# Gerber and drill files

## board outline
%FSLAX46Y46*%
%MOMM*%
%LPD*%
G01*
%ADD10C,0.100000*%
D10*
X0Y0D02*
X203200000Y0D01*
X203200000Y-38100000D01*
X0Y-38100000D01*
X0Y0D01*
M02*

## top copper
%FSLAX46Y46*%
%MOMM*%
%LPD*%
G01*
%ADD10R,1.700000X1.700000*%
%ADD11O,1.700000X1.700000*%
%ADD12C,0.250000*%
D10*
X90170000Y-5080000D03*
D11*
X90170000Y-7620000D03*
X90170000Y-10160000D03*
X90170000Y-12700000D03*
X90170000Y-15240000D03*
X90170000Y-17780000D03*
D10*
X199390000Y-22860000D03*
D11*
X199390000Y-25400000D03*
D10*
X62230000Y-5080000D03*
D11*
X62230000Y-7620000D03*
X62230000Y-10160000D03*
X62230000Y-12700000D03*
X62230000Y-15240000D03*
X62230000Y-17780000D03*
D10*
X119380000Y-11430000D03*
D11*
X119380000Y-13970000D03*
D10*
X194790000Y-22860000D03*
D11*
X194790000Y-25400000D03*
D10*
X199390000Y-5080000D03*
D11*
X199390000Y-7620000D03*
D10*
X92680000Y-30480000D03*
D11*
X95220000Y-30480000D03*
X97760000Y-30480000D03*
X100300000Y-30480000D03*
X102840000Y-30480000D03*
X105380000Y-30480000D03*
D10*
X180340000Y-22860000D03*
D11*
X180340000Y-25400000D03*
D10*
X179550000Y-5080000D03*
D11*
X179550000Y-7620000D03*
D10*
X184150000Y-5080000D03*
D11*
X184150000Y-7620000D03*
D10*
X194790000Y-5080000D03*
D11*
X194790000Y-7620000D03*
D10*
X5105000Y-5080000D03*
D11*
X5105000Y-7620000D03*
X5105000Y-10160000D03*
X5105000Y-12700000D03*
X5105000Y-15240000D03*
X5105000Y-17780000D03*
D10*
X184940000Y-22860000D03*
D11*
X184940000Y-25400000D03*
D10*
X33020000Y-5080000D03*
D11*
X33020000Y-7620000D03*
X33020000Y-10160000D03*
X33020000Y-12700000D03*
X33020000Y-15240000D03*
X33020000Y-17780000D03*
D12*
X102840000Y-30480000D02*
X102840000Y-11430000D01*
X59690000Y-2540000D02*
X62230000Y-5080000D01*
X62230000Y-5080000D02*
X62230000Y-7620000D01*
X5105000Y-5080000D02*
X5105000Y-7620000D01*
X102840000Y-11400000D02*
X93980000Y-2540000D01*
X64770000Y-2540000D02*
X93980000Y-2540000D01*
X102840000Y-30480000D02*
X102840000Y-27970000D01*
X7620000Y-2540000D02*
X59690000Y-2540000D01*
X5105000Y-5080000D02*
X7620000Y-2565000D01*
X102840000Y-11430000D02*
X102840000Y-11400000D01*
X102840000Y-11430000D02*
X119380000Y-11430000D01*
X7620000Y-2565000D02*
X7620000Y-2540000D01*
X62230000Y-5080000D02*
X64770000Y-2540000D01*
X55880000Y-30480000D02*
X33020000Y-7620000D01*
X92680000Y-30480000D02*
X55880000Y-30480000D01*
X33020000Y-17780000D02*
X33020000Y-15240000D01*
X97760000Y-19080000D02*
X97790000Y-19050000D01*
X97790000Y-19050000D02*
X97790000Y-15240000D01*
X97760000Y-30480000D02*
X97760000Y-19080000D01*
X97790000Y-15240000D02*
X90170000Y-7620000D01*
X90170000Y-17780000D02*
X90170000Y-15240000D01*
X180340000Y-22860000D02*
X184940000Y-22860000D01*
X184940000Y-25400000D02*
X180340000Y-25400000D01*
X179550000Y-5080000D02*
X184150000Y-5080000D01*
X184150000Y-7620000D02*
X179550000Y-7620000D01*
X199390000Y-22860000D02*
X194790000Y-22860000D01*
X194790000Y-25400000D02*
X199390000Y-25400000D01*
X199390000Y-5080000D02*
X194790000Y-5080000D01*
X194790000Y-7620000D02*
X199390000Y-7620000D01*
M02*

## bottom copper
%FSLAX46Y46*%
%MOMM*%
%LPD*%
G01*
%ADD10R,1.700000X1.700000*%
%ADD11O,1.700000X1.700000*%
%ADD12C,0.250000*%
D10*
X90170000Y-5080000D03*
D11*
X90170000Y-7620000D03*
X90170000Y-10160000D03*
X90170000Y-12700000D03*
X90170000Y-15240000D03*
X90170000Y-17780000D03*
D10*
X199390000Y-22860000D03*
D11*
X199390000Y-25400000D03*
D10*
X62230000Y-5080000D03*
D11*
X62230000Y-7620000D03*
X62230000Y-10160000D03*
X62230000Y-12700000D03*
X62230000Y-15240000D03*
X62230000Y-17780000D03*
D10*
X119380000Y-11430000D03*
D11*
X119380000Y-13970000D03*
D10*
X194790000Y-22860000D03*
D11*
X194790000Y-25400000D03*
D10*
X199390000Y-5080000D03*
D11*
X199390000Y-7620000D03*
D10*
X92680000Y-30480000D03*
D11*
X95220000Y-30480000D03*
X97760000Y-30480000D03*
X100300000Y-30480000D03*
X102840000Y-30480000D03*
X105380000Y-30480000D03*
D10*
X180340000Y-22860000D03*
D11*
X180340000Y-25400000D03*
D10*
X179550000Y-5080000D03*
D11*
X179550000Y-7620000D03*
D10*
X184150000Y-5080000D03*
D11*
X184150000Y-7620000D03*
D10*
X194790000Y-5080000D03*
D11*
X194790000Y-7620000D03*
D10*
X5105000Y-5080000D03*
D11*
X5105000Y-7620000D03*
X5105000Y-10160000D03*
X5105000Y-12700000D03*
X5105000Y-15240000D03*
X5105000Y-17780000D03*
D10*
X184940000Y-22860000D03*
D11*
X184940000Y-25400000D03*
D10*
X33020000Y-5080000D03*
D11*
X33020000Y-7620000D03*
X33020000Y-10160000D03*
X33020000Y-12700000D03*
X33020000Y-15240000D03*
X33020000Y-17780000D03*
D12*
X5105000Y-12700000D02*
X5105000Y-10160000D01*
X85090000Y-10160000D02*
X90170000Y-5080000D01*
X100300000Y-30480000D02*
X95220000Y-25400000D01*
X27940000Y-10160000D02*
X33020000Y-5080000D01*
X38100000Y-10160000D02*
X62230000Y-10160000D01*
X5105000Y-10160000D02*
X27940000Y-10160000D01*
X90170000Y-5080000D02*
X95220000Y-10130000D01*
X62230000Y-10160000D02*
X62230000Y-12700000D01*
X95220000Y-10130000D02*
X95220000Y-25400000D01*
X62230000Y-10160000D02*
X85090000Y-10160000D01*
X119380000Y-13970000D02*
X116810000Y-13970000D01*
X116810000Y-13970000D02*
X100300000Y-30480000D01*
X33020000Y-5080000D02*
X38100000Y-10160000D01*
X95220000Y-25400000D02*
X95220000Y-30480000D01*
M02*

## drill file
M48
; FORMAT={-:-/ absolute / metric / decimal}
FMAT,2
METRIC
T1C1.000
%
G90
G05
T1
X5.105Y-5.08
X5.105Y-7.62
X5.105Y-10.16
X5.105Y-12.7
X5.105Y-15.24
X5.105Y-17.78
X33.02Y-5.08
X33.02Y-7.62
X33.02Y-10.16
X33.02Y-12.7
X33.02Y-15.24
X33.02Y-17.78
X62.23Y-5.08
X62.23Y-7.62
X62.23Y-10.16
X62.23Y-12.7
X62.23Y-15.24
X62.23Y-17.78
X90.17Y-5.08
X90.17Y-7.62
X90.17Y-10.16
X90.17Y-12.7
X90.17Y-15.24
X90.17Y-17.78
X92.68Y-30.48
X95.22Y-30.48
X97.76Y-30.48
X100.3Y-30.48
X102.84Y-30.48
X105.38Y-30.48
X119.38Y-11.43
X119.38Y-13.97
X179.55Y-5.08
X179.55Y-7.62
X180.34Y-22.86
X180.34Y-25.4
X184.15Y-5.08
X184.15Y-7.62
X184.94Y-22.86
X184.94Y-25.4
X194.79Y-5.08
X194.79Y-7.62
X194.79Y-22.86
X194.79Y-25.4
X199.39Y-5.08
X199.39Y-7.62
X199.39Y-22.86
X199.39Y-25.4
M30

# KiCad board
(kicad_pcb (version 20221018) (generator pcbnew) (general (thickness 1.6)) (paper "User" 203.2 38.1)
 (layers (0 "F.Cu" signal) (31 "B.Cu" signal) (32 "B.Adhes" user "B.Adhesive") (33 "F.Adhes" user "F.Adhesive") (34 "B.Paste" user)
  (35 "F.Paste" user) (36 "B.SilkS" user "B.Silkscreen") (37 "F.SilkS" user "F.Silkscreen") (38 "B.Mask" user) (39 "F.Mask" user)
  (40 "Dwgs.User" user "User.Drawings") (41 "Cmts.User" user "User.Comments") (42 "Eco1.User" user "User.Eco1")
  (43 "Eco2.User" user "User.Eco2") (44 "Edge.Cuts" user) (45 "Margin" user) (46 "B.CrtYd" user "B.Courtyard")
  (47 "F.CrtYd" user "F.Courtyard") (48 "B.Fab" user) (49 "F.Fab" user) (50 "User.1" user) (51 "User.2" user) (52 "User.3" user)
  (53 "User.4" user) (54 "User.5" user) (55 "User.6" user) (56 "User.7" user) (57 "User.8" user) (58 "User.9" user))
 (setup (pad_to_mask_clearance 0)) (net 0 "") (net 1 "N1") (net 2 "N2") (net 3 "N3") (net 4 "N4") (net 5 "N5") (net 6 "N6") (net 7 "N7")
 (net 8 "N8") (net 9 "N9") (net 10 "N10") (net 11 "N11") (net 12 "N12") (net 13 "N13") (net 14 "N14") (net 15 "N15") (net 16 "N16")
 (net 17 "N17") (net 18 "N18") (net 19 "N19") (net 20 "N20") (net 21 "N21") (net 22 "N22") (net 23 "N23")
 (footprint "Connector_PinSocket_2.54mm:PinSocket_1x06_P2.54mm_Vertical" (layer "F.Cu") (at 90.17 5.08)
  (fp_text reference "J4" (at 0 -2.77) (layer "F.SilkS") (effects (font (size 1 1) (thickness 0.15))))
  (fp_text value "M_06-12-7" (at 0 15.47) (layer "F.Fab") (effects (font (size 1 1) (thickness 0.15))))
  (pad "1" thru_hole rect (at 0 0) (size 1.7 1.7) (drill 1) (layers "*.Cu" "*.Mask") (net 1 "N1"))
  (pad "2" thru_hole oval (at 0 2.54) (size 1.7 1.7) (drill 1) (layers "*.Cu" "*.Mask") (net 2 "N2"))
  (pad "3" thru_hole oval (at 0 5.08) (size 1.7 1.7) (drill 1) (layers "*.Cu" "*.Mask") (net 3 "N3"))
  (pad "4" thru_hole oval (at 0 7.62) (size 1.7 1.7) (drill 1) (layers "*.Cu" "*.Mask") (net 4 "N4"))
  (pad "5" thru_hole oval (at 0 10.16) (size 1.7 1.7) (drill 1) (layers "*.Cu" "*.Mask") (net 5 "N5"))
  (pad "6" thru_hole oval (at 0 12.7) (size 1.7 1.7) (drill 1) (layers "*.Cu" "*.Mask") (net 5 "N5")))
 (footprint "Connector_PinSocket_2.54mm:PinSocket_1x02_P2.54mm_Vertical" (layer "F.Cu") (at 199.39 22.86)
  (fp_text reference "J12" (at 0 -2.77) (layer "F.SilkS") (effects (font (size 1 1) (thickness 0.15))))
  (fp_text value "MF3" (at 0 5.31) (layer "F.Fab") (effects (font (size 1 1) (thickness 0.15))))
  (pad "1" thru_hole rect (at 0 0) (size 1.7 1.7) (drill 1) (layers "*.Cu" "*.Mask") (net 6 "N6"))
  (pad "2" thru_hole oval (at 0 2.54) (size 1.7 1.7) (drill 1) (layers "*.Cu" "*.Mask") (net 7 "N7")))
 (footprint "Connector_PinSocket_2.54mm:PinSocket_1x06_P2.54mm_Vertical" (layer "F.Cu") (at 62.23 5.08)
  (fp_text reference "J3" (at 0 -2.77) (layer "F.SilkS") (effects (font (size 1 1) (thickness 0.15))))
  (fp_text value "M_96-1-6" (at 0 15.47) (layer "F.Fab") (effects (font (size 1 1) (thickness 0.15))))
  (pad "1" thru_hole rect (at 0 0) (size 1.7 1.7) (drill 1) (layers "*.Cu" "*.Mask") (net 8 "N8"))
  (pad "2" thru_hole oval (at 0 2.54) (size 1.7 1.7) (drill 1) (layers "*.Cu" "*.Mask") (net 8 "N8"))
  (pad "3" thru_hole oval (at 0 5.08) (size 1.7 1.7) (drill 1) (layers "*.Cu" "*.Mask") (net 1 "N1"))
  (pad "4" thru_hole oval (at 0 7.62) (size 1.7 1.7) (drill 1) (layers "*.Cu" "*.Mask") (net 1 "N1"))
  (pad "5" thru_hole oval (at 0 10.16) (size 1.7 1.7) (drill 1) (layers "*.Cu" "*.Mask") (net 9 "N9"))
  (pad "6" thru_hole oval (at 0 12.7) (size 1.7 1.7) (drill 1) (layers "*.Cu" "*.Mask") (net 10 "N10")))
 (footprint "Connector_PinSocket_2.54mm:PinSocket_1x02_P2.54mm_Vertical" (layer "F.Cu") (at 119.38 11.43)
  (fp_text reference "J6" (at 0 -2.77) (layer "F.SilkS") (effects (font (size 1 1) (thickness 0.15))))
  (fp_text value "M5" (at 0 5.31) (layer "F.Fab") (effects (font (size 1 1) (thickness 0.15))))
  (pad "1" thru_hole rect (at 0 0) (size 1.7 1.7) (drill 1) (layers "*.Cu" "*.Mask") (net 8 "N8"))
  (pad "2" thru_hole oval (at 0 2.54) (size 1.7 1.7) (drill 1) (layers "*.Cu" "*.Mask") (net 1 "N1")))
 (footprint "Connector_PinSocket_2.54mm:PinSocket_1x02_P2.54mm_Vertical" (layer "F.Cu") (at 194.79 22.86)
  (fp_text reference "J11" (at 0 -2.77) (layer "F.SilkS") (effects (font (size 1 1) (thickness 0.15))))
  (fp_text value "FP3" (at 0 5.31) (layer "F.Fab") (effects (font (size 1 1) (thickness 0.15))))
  (pad "1" thru_hole rect (at 0 0) (size 1.7 1.7) (drill 1) (layers "*.Cu" "*.Mask") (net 6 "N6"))
  (pad "2" thru_hole oval (at 0 2.54) (size 1.7 1.7) (drill 1) (layers "*.Cu" "*.Mask") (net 7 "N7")))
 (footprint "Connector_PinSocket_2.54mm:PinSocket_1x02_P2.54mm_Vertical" (layer "F.Cu") (at 199.39 5.08)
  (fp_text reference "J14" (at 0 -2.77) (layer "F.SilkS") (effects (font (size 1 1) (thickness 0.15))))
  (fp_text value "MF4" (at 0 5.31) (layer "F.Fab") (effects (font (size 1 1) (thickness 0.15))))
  (pad "1" thru_hole rect (at 0 0) (size 1.7 1.7) (drill 1) (layers "*.Cu" "*.Mask") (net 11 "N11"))
  (pad "2" thru_hole oval (at 0 2.54) (size 1.7 1.7) (drill 1) (layers "*.Cu" "*.Mask") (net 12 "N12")))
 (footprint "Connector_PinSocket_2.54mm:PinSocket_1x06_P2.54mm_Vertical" (layer "F.Cu") (at 92.68 30.48 90)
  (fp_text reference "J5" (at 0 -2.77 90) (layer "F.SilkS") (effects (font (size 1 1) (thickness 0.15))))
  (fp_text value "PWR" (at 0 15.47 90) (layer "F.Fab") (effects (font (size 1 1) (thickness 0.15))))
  (pad "1" thru_hole rect (at 0 0 90) (size 1.7 1.7) (drill 1) (layers "*.Cu" "*.Mask") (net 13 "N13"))
  (pad "2" thru_hole oval (at 0 2.54 90) (size 1.7 1.7) (drill 1) (layers "*.Cu" "*.Mask") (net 1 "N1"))
  (pad "3" thru_hole oval (at 0 5.08 90) (size 1.7 1.7) (drill 1) (layers "*.Cu" "*.Mask") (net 2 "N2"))
  (pad "4" thru_hole oval (at 0 7.62 90) (size 1.7 1.7) (drill 1) (layers "*.Cu" "*.Mask") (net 1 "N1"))
  (pad "5" thru_hole oval (at 0 10.16 90) (size 1.7 1.7) (drill 1) (layers "*.Cu" "*.Mask") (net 8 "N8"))
  (pad "6" thru_hole oval (at 0 12.7 90) (size 1.7 1.7) (drill 1) (layers "*.Cu" "*.Mask") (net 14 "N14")))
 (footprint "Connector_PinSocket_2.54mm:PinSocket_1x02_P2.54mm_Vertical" (layer "F.Cu") (at 180.34 22.86)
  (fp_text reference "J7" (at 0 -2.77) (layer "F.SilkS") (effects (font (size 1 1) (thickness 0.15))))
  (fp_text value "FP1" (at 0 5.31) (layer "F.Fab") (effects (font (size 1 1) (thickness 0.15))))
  (pad "1" thru_hole rect (at 0 0) (size 1.7 1.7) (drill 1) (layers "*.Cu" "*.Mask") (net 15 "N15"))
  (pad "2" thru_hole oval (at 0 2.54) (size 1.7 1.7) (drill 1) (layers "*.Cu" "*.Mask") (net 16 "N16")))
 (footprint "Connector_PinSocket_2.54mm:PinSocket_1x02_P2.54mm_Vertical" (layer "F.Cu") (at 179.55 5.08)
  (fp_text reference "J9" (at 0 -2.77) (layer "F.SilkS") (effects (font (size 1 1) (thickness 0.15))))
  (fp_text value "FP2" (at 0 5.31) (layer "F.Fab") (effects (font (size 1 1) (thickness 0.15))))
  (pad "1" thru_hole rect (at 0 0) (size 1.7 1.7) (drill 1) (layers "*.Cu" "*.Mask") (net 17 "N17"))
  (pad "2" thru_hole oval (at 0 2.54) (size 1.7 1.7) (drill 1) (layers "*.Cu" "*.Mask") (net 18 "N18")))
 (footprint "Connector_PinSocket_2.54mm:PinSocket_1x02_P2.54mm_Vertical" (layer "F.Cu") (at 184.15 5.08)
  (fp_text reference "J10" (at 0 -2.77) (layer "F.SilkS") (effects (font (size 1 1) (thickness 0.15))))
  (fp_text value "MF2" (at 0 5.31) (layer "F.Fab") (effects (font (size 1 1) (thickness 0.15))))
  (pad "1" thru_hole rect (at 0 0) (size 1.7 1.7) (drill 1) (layers "*.Cu" "*.Mask") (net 17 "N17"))
  (pad "2" thru_hole oval (at 0 2.54) (size 1.7 1.7) (drill 1) (layers "*.Cu" "*.Mask") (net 18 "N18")))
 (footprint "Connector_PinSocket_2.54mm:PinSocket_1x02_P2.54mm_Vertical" (layer "F.Cu") (at 194.79 5.08)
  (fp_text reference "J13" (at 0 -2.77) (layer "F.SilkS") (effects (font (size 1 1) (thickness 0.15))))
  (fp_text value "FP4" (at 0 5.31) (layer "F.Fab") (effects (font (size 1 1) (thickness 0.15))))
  (pad "1" thru_hole rect (at 0 0) (size 1.7 1.7) (drill 1) (layers "*.Cu" "*.Mask") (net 11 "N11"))
  (pad "2" thru_hole oval (at 0 2.54) (size 1.7 1.7) (drill 1) (layers "*.Cu" "*.Mask") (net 12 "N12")))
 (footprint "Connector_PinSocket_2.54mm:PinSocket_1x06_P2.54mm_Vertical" (layer "F.Cu") (at 5.105 5.08)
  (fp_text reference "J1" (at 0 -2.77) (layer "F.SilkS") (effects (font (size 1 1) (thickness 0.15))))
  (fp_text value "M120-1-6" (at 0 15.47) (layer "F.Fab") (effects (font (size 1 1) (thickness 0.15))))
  (pad "1" thru_hole rect (at 0 0) (size 1.7 1.7) (drill 1) (layers "*.Cu" "*.Mask") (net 8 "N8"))
  (pad "2" thru_hole oval (at 0 2.54) (size 1.7 1.7) (drill 1) (layers "*.Cu" "*.Mask") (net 8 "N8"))
  (pad "3" thru_hole oval (at 0 5.08) (size 1.7 1.7) (drill 1) (layers "*.Cu" "*.Mask") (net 1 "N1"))
  (pad "4" thru_hole oval (at 0 7.62) (size 1.7 1.7) (drill 1) (layers "*.Cu" "*.Mask") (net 1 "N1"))
  (pad "5" thru_hole oval (at 0 10.16) (size 1.7 1.7) (drill 1) (layers "*.Cu" "*.Mask") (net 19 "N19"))
  (pad "6" thru_hole oval (at 0 12.7) (size 1.7 1.7) (drill 1) (layers "*.Cu" "*.Mask") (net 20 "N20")))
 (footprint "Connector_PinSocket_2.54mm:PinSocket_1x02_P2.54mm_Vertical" (layer "F.Cu") (at 184.94 22.86)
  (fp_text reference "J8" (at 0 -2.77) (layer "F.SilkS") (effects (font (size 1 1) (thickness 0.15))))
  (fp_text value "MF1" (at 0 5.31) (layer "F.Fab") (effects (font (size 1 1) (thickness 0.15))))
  (pad "1" thru_hole rect (at 0 0) (size 1.7 1.7) (drill 1) (layers "*.Cu" "*.Mask") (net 15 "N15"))
  (pad "2" thru_hole oval (at 0 2.54) (size 1.7 1.7) (drill 1) (layers "*.Cu" "*.Mask") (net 16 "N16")))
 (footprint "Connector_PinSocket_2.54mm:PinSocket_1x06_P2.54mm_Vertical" (layer "F.Cu") (at 33.02 5.08)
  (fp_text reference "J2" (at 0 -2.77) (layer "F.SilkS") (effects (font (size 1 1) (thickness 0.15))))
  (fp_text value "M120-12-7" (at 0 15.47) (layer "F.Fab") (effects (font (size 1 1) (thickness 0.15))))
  (pad "1" thru_hole rect (at 0 0) (size 1.7 1.7) (drill 1) (layers "*.Cu" "*.Mask") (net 1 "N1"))
  (pad "2" thru_hole oval (at 0 2.54) (size 1.7 1.7) (drill 1) (layers "*.Cu" "*.Mask") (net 13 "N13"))
  (pad "3" thru_hole oval (at 0 5.08) (size 1.7 1.7) (drill 1) (layers "*.Cu" "*.Mask") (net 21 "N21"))
  (pad "4" thru_hole oval (at 0 7.62) (size 1.7 1.7) (drill 1) (layers "*.Cu" "*.Mask") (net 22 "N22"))
  (pad "5" thru_hole oval (at 0 10.16) (size 1.7 1.7) (drill 1) (layers "*.Cu" "*.Mask") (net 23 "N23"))
  (pad "6" thru_hole oval (at 0 12.7) (size 1.7 1.7) (drill 1) (layers "*.Cu" "*.Mask") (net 23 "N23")))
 (gr_rect (start 0 0) (end 203.2 38.1) (stroke (width 0.1) (type default)) (fill none) (layer "Edge.Cuts"))
 (segment (start 102.84 30.48) (end 102.84 11.43) (width 0.25) (layer "F.Cu") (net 8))
 (segment (start 59.69 2.54) (end 62.23 5.08) (width 0.25) (layer "F.Cu") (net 8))
 (segment (start 62.23 5.08) (end 62.23 7.62) (width 0.25) (layer "F.Cu") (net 8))
 (segment (start 5.105 5.08) (end 5.105 7.62) (width 0.25) (layer "F.Cu") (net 8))
 (segment (start 102.84 11.4) (end 93.98 2.54) (width 0.25) (layer "F.Cu") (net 8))
 (segment (start 64.77 2.54) (end 93.98 2.54) (width 0.25) (layer "F.Cu") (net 8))
 (segment (start 102.84 30.48) (end 102.84 27.97) (width 0.25) (layer "F.Cu") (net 8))
 (segment (start 7.62 2.54) (end 59.69 2.54) (width 0.25) (layer "F.Cu") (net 8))
 (segment (start 5.105 5.08) (end 7.62 2.565) (width 0.25) (layer "F.Cu") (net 8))
 (segment (start 102.84 11.43) (end 102.84 11.4) (width 0.25) (layer "F.Cu") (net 8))
 (segment (start 102.84 11.43) (end 119.38 11.43) (width 0.25) (layer "F.Cu") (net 8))
 (segment (start 7.62 2.565) (end 7.62 2.54) (width 0.25) (layer "F.Cu") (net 8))
 (segment (start 62.23 5.08) (end 64.77 2.54) (width 0.25) (layer "F.Cu") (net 8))
 (segment (start 5.105 12.7) (end 5.105 10.16) (width 0.25) (layer "B.Cu") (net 1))
 (segment (start 85.09 10.16) (end 90.17 5.08) (width 0.25) (layer "B.Cu") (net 1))
 (segment (start 100.3 30.48) (end 95.22 25.4) (width 0.25) (layer "B.Cu") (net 1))
 (segment (start 27.94 10.16) (end 33.02 5.08) (width 0.25) (layer "B.Cu") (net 1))
 (segment (start 38.1 10.16) (end 62.23 10.16) (width 0.25) (layer "B.Cu") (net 1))
 (segment (start 5.105 10.16) (end 27.94 10.16) (width 0.25) (layer "B.Cu") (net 1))
 (segment (start 90.17 5.08) (end 95.22 10.13) (width 0.25) (layer "B.Cu") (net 1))
 (segment (start 62.23 10.16) (end 62.23 12.7) (width 0.25) (layer "B.Cu") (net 1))
 (segment (start 95.22 10.13) (end 95.22 25.4) (width 0.25) (layer "B.Cu") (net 1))
 (segment (start 62.23 10.16) (end 85.09 10.16) (width 0.25) (layer "B.Cu") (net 1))
 (segment (start 119.38 13.97) (end 116.81 13.97) (width 0.25) (layer "B.Cu") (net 1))
 (segment (start 116.81 13.97) (end 100.3 30.48) (width 0.25) (layer "B.Cu") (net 1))
 (segment (start 33.02 5.08) (end 38.1 10.16) (width 0.25) (layer "B.Cu") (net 1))
 (segment (start 95.22 25.4) (end 95.22 30.48) (width 0.25) (layer "B.Cu") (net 1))
 (segment (start 55.88 30.48) (end 33.02 7.62) (width 0.25) (layer "F.Cu") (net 13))
 (segment (start 92.68 30.48) (end 55.88 30.48) (width 0.25) (layer "F.Cu") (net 13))
 (segment (start 33.02 17.78) (end 33.02 15.24) (width 0.25) (layer "F.Cu") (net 23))
 (segment (start 97.76 19.08) (end 97.79 19.05) (width 0.25) (layer "F.Cu") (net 2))
 (segment (start 97.79 19.05) (end 97.79 15.24) (width 0.25) (layer "F.Cu") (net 2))
 (segment (start 97.76 30.48) (end 97.76 19.08) (width 0.25) (layer "F.Cu") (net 2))
 (segment (start 97.79 15.24) (end 90.17 7.62) (width 0.25) (layer "F.Cu") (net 2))
 (segment (start 90.17 17.78) (end 90.17 15.24) (width 0.25) (layer "F.Cu") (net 5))
 (segment (start 180.34 22.86) (end 184.94 22.86) (width 0.25) (layer "F.Cu") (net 15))
 (segment (start 184.94 25.4) (end 180.34 25.4) (width 0.25) (layer "F.Cu") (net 16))
 (segment (start 179.55 5.08) (end 184.15 5.08) (width 0.25) (layer "F.Cu") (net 17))
 (segment (start 184.15 7.62) (end 179.55 7.62) (width 0.25) (layer "F.Cu") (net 18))
 (segment (start 199.39 22.86) (end 194.79 22.86) (width 0.25) (layer "F.Cu") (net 6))
 (segment (start 194.79 25.4) (end 199.39 25.4) (width 0.25) (layer "F.Cu") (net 7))
 (segment (start 199.39 5.08) (end 194.79 5.08) (width 0.25) (layer "F.Cu") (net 11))
 (segment (start 194.79 7.62) (end 199.39 7.62) (width 0.25) (layer "F.Cu") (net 12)))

